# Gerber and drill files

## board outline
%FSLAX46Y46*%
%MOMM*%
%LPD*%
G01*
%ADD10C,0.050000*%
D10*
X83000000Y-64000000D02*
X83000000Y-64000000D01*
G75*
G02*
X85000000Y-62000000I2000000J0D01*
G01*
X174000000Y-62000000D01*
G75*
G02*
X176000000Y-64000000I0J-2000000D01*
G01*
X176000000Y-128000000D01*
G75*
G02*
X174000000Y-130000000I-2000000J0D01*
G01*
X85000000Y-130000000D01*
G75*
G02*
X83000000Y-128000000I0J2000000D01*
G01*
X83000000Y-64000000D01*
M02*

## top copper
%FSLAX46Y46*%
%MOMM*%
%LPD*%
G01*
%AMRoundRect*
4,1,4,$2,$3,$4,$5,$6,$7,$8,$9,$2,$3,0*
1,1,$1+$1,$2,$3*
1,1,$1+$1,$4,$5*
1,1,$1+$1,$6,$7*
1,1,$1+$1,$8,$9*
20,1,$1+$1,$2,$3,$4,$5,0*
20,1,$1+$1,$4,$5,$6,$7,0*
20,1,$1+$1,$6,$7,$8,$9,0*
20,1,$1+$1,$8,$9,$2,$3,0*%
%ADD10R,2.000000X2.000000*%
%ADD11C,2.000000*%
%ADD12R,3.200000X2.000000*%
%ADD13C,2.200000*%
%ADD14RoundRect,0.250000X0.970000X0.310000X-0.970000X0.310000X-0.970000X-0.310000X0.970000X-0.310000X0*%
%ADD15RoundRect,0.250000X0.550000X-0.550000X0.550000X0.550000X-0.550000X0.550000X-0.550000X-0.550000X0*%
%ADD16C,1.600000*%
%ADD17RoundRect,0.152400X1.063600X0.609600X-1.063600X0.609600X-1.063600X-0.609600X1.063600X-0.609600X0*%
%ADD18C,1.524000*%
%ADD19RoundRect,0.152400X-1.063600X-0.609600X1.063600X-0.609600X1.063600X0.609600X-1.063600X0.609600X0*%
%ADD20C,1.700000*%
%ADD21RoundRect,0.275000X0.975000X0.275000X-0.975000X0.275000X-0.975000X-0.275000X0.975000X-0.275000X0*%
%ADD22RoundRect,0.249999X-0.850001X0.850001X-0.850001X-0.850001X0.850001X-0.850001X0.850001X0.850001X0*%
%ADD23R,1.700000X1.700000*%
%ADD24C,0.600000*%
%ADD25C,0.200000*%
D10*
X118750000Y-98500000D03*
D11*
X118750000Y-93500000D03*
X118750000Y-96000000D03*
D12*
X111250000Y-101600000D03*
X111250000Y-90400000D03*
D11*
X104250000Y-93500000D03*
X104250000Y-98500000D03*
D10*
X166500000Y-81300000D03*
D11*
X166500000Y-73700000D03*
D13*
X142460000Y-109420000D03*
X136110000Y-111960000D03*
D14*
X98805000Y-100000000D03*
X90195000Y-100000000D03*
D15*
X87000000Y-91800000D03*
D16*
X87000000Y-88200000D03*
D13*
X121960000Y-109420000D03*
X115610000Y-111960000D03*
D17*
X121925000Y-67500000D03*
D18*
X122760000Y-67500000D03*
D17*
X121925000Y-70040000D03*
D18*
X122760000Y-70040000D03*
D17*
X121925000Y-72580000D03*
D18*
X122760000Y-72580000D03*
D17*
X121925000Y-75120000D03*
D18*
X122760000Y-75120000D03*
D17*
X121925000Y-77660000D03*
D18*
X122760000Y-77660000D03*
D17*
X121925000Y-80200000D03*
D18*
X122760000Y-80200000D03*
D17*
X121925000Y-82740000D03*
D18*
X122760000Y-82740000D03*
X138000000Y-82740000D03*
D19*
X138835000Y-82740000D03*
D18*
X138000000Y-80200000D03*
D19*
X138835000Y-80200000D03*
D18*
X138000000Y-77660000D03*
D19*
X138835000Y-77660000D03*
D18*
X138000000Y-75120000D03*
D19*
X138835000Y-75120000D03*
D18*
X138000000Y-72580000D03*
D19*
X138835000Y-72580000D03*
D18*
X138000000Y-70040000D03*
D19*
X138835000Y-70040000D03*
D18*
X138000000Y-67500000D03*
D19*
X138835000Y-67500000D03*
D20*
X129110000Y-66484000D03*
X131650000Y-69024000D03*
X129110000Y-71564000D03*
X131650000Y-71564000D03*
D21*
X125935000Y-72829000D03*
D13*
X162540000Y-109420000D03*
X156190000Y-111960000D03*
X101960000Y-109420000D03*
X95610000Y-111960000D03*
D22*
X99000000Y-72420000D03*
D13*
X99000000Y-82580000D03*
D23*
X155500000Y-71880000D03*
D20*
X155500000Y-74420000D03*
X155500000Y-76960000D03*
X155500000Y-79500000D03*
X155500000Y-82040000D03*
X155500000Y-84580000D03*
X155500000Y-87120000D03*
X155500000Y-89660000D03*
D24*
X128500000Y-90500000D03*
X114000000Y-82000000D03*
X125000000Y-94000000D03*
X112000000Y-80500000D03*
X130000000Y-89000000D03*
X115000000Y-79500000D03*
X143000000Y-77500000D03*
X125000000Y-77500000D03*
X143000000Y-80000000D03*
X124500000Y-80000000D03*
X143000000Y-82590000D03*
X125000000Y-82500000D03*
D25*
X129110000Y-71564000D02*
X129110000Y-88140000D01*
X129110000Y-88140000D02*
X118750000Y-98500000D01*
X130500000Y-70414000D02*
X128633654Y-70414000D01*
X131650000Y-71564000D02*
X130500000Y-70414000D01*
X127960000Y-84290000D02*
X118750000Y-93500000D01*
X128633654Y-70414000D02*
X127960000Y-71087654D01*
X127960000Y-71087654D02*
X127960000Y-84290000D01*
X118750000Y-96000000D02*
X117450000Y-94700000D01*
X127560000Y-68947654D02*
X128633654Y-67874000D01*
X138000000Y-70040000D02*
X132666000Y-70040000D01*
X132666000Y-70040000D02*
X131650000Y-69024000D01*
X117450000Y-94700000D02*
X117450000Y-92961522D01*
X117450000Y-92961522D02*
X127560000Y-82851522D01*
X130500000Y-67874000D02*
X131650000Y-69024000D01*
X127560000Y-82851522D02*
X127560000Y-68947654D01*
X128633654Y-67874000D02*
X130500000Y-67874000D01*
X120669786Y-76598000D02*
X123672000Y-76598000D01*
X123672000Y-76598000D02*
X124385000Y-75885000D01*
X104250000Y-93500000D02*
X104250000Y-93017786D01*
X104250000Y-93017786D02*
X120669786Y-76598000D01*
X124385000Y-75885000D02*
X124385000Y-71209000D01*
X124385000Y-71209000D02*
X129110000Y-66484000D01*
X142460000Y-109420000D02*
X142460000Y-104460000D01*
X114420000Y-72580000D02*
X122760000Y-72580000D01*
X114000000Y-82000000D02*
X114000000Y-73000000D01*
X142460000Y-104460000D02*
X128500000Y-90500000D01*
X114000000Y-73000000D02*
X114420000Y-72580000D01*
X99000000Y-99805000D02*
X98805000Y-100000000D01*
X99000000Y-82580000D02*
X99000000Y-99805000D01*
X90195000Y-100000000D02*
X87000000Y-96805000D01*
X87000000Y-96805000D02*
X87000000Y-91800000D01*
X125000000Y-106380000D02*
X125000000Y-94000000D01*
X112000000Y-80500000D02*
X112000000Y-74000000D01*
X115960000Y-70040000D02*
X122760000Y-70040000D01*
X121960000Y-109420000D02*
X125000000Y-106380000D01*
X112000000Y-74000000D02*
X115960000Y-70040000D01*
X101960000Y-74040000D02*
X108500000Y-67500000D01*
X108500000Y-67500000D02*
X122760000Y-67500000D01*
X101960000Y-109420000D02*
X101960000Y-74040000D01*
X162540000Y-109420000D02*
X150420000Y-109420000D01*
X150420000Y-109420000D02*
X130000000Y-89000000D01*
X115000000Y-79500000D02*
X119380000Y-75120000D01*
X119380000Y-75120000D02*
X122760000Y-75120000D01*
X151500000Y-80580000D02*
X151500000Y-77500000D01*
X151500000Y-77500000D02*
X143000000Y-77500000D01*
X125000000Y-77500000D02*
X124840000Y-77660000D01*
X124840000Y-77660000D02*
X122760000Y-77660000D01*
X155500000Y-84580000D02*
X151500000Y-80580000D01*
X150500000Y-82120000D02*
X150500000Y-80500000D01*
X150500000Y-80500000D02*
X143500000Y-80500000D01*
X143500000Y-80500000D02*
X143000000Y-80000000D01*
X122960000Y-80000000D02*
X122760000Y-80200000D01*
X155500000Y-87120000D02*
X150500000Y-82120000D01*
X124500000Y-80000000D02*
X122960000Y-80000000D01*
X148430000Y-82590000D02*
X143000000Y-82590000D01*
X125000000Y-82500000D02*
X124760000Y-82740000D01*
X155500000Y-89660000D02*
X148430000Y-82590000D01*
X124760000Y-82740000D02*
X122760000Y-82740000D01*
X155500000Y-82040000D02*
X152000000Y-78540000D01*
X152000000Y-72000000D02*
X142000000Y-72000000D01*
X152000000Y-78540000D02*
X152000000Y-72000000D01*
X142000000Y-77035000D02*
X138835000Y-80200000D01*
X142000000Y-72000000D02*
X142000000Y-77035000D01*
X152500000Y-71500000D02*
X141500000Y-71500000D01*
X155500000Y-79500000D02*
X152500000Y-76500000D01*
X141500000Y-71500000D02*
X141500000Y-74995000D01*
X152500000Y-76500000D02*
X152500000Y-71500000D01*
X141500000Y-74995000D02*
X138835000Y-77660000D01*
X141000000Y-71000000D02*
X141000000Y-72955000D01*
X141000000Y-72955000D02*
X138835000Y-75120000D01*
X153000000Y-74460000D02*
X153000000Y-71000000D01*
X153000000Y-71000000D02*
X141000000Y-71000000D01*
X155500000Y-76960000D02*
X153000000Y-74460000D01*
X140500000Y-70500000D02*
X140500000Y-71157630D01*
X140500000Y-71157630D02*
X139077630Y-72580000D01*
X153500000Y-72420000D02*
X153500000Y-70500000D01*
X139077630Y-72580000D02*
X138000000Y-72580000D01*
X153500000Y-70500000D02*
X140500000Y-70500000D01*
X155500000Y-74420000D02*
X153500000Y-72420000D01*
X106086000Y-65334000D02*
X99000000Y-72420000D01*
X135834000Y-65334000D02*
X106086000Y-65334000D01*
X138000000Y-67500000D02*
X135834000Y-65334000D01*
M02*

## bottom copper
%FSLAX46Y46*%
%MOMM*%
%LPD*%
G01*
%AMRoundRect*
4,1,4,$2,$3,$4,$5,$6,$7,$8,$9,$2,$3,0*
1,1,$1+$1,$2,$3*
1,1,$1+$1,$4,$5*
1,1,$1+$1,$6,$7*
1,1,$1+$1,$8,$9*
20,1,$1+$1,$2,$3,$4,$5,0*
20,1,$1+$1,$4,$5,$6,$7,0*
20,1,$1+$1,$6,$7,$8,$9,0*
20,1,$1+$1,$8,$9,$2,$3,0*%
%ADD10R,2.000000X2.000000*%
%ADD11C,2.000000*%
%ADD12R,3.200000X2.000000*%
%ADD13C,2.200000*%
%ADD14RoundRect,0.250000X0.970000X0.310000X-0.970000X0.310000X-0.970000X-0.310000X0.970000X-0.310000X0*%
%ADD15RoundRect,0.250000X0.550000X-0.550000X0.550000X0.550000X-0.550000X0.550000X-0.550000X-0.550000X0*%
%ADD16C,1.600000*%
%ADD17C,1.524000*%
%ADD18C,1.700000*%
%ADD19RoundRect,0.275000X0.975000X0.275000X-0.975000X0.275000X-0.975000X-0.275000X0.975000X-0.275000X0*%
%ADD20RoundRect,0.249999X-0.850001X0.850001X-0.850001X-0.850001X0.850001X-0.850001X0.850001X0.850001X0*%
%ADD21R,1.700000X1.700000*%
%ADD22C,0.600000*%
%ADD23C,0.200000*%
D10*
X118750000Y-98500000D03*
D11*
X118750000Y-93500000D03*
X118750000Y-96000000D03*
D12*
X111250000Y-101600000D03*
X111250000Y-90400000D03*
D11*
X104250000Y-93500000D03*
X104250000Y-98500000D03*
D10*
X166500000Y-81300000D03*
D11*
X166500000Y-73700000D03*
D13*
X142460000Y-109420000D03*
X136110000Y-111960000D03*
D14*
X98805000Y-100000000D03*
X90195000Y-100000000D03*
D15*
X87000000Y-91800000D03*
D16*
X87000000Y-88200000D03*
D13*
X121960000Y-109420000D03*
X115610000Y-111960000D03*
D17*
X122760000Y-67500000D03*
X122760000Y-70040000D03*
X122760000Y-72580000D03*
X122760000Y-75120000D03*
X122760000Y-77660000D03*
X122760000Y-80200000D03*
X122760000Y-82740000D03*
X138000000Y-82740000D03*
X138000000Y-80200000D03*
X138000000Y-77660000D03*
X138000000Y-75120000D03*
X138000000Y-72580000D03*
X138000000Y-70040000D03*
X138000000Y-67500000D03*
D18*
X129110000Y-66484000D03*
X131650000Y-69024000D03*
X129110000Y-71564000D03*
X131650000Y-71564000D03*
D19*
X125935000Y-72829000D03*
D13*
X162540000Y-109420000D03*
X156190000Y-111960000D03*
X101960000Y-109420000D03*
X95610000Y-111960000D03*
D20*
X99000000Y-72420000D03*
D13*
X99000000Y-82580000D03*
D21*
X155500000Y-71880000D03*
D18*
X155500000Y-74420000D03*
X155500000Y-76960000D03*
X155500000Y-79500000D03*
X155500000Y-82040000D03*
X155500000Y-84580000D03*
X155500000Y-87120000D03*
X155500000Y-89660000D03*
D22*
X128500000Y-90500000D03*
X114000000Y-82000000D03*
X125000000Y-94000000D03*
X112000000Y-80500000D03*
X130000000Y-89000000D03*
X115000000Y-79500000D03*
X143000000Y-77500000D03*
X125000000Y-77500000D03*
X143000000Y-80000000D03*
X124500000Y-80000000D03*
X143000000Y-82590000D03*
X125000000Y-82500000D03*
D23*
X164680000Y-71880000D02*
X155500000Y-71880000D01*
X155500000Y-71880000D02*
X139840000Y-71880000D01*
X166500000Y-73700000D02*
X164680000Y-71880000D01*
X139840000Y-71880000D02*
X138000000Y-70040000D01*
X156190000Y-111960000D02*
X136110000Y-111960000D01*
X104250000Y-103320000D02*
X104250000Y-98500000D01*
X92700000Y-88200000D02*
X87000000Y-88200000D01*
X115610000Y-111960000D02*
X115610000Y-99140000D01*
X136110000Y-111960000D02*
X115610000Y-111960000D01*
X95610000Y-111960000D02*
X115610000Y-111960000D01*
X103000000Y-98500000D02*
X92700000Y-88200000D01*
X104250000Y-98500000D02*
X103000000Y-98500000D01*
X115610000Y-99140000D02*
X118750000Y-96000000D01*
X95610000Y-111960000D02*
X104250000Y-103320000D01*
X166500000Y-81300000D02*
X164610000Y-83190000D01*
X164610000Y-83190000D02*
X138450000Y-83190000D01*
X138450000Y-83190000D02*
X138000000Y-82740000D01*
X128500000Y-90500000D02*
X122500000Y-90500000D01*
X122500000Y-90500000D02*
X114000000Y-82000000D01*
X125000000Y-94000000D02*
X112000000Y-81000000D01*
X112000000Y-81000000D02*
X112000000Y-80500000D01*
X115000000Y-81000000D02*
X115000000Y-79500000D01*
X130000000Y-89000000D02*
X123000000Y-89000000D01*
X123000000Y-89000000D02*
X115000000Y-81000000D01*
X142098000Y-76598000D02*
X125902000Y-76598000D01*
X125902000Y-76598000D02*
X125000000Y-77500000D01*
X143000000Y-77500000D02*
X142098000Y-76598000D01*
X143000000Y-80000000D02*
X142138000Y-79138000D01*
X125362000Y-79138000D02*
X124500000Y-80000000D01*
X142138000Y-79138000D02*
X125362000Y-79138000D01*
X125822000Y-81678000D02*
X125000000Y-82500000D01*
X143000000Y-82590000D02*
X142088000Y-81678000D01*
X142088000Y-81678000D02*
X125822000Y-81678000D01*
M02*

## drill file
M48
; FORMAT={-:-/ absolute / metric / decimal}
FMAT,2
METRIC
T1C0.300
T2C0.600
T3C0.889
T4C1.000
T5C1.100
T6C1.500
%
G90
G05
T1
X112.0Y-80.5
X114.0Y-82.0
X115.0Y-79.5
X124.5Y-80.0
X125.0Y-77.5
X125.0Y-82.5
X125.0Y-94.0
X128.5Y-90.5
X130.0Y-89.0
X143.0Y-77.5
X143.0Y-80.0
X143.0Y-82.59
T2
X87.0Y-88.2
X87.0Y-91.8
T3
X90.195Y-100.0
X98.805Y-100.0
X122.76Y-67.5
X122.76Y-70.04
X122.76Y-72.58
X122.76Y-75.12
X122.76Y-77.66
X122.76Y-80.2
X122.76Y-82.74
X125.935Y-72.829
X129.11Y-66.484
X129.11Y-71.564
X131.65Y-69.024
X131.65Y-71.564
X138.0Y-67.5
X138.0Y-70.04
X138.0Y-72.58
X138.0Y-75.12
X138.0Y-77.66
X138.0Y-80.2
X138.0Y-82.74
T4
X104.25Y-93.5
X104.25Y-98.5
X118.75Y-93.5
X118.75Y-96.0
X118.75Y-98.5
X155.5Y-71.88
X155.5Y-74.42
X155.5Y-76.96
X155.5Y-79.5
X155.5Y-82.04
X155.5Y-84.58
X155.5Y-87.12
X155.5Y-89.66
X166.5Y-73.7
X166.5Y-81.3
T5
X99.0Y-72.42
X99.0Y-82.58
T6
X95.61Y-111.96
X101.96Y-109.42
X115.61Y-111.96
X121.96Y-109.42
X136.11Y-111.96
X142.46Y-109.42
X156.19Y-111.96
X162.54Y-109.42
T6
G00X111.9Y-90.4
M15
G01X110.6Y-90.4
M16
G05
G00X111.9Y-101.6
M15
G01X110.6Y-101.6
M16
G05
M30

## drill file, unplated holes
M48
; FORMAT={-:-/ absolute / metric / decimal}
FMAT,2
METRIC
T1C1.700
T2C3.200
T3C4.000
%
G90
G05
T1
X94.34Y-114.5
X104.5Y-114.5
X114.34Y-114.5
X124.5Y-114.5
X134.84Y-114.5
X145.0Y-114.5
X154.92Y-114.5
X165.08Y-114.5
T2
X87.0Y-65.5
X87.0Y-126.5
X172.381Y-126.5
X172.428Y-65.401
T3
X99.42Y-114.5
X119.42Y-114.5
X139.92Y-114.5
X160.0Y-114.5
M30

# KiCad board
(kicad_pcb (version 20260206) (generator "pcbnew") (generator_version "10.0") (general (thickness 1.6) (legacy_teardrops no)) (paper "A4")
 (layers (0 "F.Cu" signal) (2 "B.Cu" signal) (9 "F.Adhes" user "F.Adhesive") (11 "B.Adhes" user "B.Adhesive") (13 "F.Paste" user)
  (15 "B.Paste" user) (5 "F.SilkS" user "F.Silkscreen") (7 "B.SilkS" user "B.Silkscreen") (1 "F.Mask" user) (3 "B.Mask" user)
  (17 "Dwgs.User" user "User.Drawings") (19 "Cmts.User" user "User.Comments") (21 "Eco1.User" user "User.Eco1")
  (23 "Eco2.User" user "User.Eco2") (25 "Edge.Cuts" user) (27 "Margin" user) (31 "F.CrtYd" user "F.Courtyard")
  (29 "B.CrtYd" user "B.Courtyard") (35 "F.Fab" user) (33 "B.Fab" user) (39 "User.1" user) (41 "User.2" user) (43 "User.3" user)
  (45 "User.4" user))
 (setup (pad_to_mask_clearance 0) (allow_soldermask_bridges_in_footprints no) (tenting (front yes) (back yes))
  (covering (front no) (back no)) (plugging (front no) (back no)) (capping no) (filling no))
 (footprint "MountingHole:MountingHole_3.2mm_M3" (layer "F.Cu") (at 172.380609 126.5)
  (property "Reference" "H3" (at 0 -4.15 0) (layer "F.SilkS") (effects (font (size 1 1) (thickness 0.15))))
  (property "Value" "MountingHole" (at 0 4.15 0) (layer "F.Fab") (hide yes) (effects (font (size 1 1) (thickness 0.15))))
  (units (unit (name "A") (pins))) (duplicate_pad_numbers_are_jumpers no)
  (pad "" np_thru_hole circle (at 0 0) (size 3.2 3.2) (drill 3.2) (layers "*.Cu" "*.Mask")))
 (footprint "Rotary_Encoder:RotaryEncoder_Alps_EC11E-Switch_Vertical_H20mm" (layer "F.Cu") (at 118.75 98.5 180)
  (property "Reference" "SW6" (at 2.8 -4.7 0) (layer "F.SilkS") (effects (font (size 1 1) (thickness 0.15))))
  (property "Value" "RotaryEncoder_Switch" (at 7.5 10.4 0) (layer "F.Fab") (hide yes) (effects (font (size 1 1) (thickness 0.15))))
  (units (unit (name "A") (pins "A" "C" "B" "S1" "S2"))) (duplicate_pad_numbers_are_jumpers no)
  (pad "A" thru_hole rect (at 0 0 180) (size 2 2) (drill 1) (layers "*.Cu" "*.Mask") (remove_unused_layers no)
   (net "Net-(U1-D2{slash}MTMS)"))
  (pad "B" thru_hole circle (at 0 5 180) (size 2 2) (drill 1) (layers "*.Cu" "*.Mask") (remove_unused_layers no)
   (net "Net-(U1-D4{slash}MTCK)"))
  (pad "C" thru_hole circle (at 0 2.5 180) (size 2 2) (drill 1) (layers "*.Cu" "*.Mask") (remove_unused_layers no) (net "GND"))
  (pad "MP" thru_hole rect (at 7.5 -3.1 180) (size 3.2 2) (drill oval 2.8 1.5) (layers "*.Cu" "*.Mask") (remove_unused_layers no))
  (pad "MP" thru_hole rect (at 7.5 8.1 180) (size 3.2 2) (drill oval 2.8 1.5) (layers "*.Cu" "*.Mask") (remove_unused_layers no))
  (pad "S1" thru_hole circle (at 14.5 5 180) (size 2 2) (drill 1) (layers "*.Cu" "*.Mask") (remove_unused_layers no)
   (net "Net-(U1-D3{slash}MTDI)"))
  (pad "S2" thru_hole circle (at 14.5 0 180) (size 2 2) (drill 1) (layers "*.Cu" "*.Mask") (remove_unused_layers no) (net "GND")))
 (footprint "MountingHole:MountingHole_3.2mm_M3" (layer "F.Cu") (at 172.4285 65.401372)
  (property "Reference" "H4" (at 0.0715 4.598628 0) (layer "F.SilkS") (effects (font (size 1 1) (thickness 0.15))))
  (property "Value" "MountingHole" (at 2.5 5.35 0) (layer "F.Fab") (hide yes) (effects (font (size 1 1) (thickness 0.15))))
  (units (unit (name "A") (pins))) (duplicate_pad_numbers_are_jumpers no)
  (pad "" np_thru_hole circle (at 0 0) (size 3.2 3.2) (drill 3.2) (layers "*.Cu" "*.Mask")))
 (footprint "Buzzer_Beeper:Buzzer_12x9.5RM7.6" (layer "F.Cu") (at 166.5 81.3 90)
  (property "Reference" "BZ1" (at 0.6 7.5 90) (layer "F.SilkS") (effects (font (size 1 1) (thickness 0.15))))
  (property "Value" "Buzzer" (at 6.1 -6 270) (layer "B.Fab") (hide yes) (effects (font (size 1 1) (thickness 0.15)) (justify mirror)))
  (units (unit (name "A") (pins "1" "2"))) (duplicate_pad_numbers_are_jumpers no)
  (pad "1" thru_hole rect (at 0 0 90) (size 2 2) (drill 1) (layers "*.Cu" "*.Mask") (remove_unused_layers no) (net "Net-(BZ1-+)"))
  (pad "2" thru_hole circle (at 7.6 0 90) (size 2 2) (drill 1) (layers "*.Cu" "*.Mask") (remove_unused_layers no) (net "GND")))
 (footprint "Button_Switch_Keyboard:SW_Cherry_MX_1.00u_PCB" (layer "F.Cu") (at 142.46 109.42)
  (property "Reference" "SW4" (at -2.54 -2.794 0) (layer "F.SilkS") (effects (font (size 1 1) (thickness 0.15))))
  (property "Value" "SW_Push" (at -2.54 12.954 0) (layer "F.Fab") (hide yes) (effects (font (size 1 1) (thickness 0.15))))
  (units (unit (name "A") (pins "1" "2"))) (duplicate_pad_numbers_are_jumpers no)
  (pad "" np_thru_hole circle (at -7.62 5.08) (size 1.7 1.7) (drill 1.7) (layers "*.Cu" "*.Mask"))
  (pad "" np_thru_hole circle (at -2.54 5.08) (size 4 4) (drill 4) (layers "*.Cu" "*.Mask"))
  (pad "" np_thru_hole circle (at 2.54 5.08) (size 1.7 1.7) (drill 1.7) (layers "*.Cu" "*.Mask"))
  (pad "1" thru_hole circle (at 0 0) (size 2.2 2.2) (drill 1.5) (layers "*.Cu" "*.Mask") (remove_unused_layers no) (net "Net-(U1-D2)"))
  (pad "2" thru_hole circle (at -6.35 2.54) (size 2.2 2.2) (drill 1.5) (layers "*.Cu" "*.Mask") (remove_unused_layers no) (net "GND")))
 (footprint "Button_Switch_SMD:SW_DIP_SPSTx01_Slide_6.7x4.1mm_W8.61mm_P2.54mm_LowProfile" (layer "F.Cu") (at 94.5 100 180)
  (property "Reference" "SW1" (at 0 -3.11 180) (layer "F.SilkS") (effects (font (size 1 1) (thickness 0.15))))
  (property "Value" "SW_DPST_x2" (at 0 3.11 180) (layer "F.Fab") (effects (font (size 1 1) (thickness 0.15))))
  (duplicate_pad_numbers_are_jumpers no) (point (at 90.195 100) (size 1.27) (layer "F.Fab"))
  (pad "1" thru_hole roundrect (at -4.305 0 180) (size 2.44 1.12) (drill 0.889) (layers "*.Cu" "*.Mask" "F.Paste") (remove_unused_layers no)
   (roundrect_rratio 0.223214) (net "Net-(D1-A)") (zone_connect 2))
  (pad "2" thru_hole roundrect (at 4.305 0 180) (size 2.44 1.12) (drill 0.889) (layers "*.Cu" "*.Mask") (remove_unused_layers no)
   (roundrect_rratio 0.223214) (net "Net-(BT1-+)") (zone_connect 2)))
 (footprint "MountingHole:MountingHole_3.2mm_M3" (layer "F.Cu") (at 87 126.5)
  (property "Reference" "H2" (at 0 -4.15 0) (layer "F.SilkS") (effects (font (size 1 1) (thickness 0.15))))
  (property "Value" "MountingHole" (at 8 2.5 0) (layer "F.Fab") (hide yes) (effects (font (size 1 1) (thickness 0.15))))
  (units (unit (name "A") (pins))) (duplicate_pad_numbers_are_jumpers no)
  (pad "" np_thru_hole circle (at 0 0) (size 3.2 3.2) (drill 3.2) (layers "*.Cu" "*.Mask")))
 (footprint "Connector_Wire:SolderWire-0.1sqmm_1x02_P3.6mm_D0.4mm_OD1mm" (layer "F.Cu") (at 87 91.8 90)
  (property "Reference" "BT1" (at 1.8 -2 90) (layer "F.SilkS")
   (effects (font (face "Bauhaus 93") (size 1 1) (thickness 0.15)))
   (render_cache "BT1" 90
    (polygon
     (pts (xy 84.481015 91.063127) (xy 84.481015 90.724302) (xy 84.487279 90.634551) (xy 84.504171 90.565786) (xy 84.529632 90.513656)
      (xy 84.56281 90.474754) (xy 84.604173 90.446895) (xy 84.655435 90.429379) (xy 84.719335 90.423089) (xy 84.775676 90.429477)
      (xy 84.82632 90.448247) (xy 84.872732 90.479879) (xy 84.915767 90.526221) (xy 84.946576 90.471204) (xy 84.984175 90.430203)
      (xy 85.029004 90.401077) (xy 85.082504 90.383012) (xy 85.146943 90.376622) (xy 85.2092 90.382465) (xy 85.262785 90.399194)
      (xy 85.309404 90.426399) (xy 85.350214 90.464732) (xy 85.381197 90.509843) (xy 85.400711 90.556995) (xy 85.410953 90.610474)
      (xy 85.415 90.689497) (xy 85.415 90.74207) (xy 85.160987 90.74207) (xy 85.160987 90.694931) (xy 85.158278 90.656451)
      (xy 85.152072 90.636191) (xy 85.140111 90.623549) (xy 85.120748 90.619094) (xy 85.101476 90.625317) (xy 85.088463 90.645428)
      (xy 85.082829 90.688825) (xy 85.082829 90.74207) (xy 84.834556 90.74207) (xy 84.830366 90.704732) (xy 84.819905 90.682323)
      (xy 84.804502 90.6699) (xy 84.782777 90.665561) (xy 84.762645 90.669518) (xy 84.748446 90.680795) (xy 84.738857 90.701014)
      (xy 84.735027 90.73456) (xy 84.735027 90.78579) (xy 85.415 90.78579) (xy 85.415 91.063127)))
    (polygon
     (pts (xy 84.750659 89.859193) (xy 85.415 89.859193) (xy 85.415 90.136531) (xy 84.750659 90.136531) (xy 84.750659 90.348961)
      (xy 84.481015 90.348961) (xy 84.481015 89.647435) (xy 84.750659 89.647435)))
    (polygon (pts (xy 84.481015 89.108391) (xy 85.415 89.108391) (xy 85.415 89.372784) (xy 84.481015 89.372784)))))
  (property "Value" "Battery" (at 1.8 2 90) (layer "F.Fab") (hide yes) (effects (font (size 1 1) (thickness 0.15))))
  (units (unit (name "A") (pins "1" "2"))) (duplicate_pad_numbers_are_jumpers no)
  (pad "1" thru_hole roundrect (at 0 0 90) (size 1.6 1.6) (drill 0.6) (layers "*.Cu" "*.Mask") (remove_unused_layers no)
   (roundrect_rratio 0.15625) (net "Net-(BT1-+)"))
  (pad "2" thru_hole circle (at 3.6 0 90) (size 1.6 1.6) (drill 0.6) (layers "*.Cu" "*.Mask") (remove_unused_layers no) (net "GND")))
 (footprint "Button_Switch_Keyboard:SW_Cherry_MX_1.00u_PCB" (layer "F.Cu") (at 121.96 109.42)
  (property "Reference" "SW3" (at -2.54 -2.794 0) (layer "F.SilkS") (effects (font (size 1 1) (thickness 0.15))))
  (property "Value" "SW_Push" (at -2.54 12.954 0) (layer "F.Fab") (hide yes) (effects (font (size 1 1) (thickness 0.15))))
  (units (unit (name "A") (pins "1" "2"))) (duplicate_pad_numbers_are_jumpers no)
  (pad "" np_thru_hole circle (at -7.62 5.08) (size 1.7 1.7) (drill 1.7) (layers "*.Cu" "*.Mask"))
  (pad "" np_thru_hole circle (at -2.54 5.08) (size 4 4) (drill 4) (layers "*.Cu" "*.Mask"))
  (pad "" np_thru_hole circle (at 2.54 5.08) (size 1.7 1.7) (drill 1.7) (layers "*.Cu" "*.Mask"))
  (pad "1" thru_hole circle (at 0 0) (size 2.2 2.2) (drill 1.5) (layers "*.Cu" "*.Mask") (remove_unused_layers no) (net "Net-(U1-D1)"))
  (pad "2" thru_hole circle (at -6.35 2.54) (size 2.2 2.2) (drill 1.5) (layers "*.Cu" "*.Mask") (remove_unused_layers no) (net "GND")))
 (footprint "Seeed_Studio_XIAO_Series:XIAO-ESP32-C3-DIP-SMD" (layer "F.Cu") (at 130.38 75.12 90)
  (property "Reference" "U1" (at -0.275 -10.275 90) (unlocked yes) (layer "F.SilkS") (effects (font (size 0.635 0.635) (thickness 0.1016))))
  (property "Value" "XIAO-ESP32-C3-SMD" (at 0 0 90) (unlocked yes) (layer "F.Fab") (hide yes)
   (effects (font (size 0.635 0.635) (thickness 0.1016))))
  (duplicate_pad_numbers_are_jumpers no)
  (pad "1" smd roundrect (at 7.62 -8.455 180) (size 2.432 1.524) (layers "F.Cu" "F.Mask") (roundrect_rratio 0.1) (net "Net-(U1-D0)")
   (thermal_bridge_angle 45))
  (pad "1" thru_hole circle (at 7.62 -7.62 180) (size 1.524 1.524) (drill 0.889) (layers "*.Cu" "*.Mask") (remove_unused_layers no)
   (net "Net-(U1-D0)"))
  (pad "2" smd roundrect (at 5.08 -8.455 180) (size 2.432 1.524) (layers "F.Cu" "F.Mask") (roundrect_rratio 0.1) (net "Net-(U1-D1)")
   (thermal_bridge_angle 45))
  (pad "2" thru_hole circle (at 5.08 -7.62 180) (size 1.524 1.524) (drill 0.889) (layers "*.Cu" "*.Mask") (remove_unused_layers no)
   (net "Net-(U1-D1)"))
  (pad "3" smd roundrect (at 2.54 -8.455 180) (size 2.432 1.524) (layers "F.Cu" "F.Mask") (roundrect_rratio 0.1) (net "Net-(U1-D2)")
   (thermal_bridge_angle 45))
  (pad "3" thru_hole circle (at 2.54 -7.62 180) (size 1.524 1.524) (drill 0.889) (layers "*.Cu" "*.Mask") (remove_unused_layers no)
   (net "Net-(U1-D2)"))
  (pad "4" smd roundrect (at 0 -8.455 180) (size 2.432 1.524) (layers "F.Cu" "F.Mask") (roundrect_rratio 0.1) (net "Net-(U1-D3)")
   (thermal_bridge_angle 45))
  (pad "4" thru_hole circle (at 0 -7.62 180) (size 1.524 1.524) (drill 0.889) (layers "*.Cu" "*.Mask") (remove_unused_layers no)
   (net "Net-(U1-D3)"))
  (pad "5" smd roundrect (at -2.54 -8.455 180) (size 2.432 1.524) (layers "F.Cu" "F.Mask") (roundrect_rratio 0.1) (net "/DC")
   (thermal_bridge_angle 45))
  (pad "5" thru_hole circle (at -2.54 -7.62 180) (size 1.524 1.524) (drill 0.889) (layers "*.Cu" "*.Mask") (remove_unused_layers no)
   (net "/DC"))
  (pad "6" smd roundrect (at -5.08 -8.455 180) (size 2.432 1.524) (layers "F.Cu" "F.Mask") (roundrect_rratio 0.1) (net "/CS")
   (thermal_bridge_angle 45))
  (pad "6" thru_hole circle (at -5.08 -7.62 180) (size 1.524 1.524) (drill 0.889) (layers "*.Cu" "*.Mask") (remove_unused_layers no)
   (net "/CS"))
  (pad "7" smd roundrect (at -7.62 -8.455 180) (size 2.432 1.524) (layers "F.Cu" "F.Mask") (roundrect_rratio 0.1) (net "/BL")
   (thermal_bridge_angle 45))
  (pad "7" thru_hole circle (at -7.62 -7.62 180) (size 1.524 1.524) (drill 0.889) (layers "*.Cu" "*.Mask") (remove_unused_layers no)
   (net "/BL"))
  (pad "8" thru_hole circle (at -7.62 7.62) (size 1.524 1.524) (drill 0.889) (layers "*.Cu" "*.Mask") (remove_unused_layers no)
   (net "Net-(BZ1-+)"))
  (pad "8" smd roundrect (at -7.62 8.455) (size 2.432 1.524) (layers "F.Cu" "F.Mask") (roundrect_rratio 0.1) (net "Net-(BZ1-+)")
   (thermal_bridge_angle 45))
  (pad "9" thru_hole circle (at -5.08 7.62) (size 1.524 1.524) (drill 0.889) (layers "*.Cu" "*.Mask") (remove_unused_layers no) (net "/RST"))
  (pad "9" smd roundrect (at -5.08 8.455) (size 2.432 1.524) (layers "F.Cu" "F.Mask") (roundrect_rratio 0.1) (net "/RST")
   (thermal_bridge_angle 45))
  (pad "10" thru_hole circle (at -2.54 7.62) (size 1.524 1.524) (drill 0.889) (layers "*.Cu" "*.Mask") (remove_unused_layers no)
   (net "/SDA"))
  (pad "10" smd roundrect (at -2.54 8.455) (size 2.432 1.524) (layers "F.Cu" "F.Mask") (roundrect_rratio 0.1) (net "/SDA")
   (thermal_bridge_angle 45))
  (pad "11" thru_hole circle (at 0 7.62) (size 1.524 1.524) (drill 0.889) (layers "*.Cu" "*.Mask") (remove_unused_layers no) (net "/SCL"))
  (pad "11" smd roundrect (at 0 8.455) (size 2.432 1.524) (layers "F.Cu" "F.Mask") (roundrect_rratio 0.1) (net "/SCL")
   (thermal_bridge_angle 45))
  (pad "12" thru_hole circle (at 2.54 7.62) (size 1.524 1.524) (drill 0.889) (layers "*.Cu" "*.Mask") (remove_unused_layers no)
   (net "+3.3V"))
  (pad "12" smd roundrect (at 2.54 8.455) (size 2.432 1.524) (layers "F.Cu" "F.Mask") (roundrect_rratio 0.1) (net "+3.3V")
   (thermal_bridge_angle 45))
  (pad "13" thru_hole circle (at 5.08 7.62) (size 1.524 1.524) (drill 0.889) (layers "*.Cu" "*.Mask") (remove_unused_layers no) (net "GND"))
  (pad "13" smd roundrect (at 5.08 8.455) (size 2.432 1.524) (layers "F.Cu" "F.Mask") (roundrect_rratio 0.1) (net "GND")
   (thermal_bridge_angle 45))
  (pad "14" thru_hole circle (at 7.62 7.62) (size 1.524 1.524) (drill 0.889) (layers "*.Cu" "*.Mask") (remove_unused_layers no)
   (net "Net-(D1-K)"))
  (pad "14" smd roundrect (at 7.62 8.455) (size 2.432 1.524) (layers "F.Cu" "F.Mask") (roundrect_rratio 0.1) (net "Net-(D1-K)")
   (thermal_bridge_angle 45))
  (pad "15" thru_hole circle (at 8.636 -1.27) (size 1.7 1.7) (drill 0.889) (layers "*.Cu" "*.Mask") (remove_unused_layers no)
   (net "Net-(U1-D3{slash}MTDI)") (zone_connect 2))
  (pad "18" thru_hole circle (at 6.096 1.27) (size 1.7 1.7) (drill 0.889) (layers "*.Cu" "*.Mask") (remove_unused_layers no) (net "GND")
   (zone_connect 2))
  (pad "19" thru_hole circle (at 3.556 -1.27) (size 1.7 1.7) (drill 0.889) (layers "*.Cu" "*.Mask") (remove_unused_layers no)
   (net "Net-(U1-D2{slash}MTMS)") (zone_connect 2))
  (pad "20" thru_hole circle (at 3.556 1.27) (size 1.7 1.7) (drill 0.889) (layers "*.Cu" "F.Mask") (remove_unused_layers no)
   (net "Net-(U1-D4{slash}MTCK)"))
  (pad "GND" thru_hole roundrect (at 2.291 -4.445 180) (size 2.5 1.1) (drill 0.889) (layers "*.Cu" "*.Mask") (remove_unused_layers no)
   (roundrect_rratio 0.25) (die_length 2) (thermal_bridge_angle 45)))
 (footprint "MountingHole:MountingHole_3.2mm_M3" (layer "F.Cu") (at 87 65.5)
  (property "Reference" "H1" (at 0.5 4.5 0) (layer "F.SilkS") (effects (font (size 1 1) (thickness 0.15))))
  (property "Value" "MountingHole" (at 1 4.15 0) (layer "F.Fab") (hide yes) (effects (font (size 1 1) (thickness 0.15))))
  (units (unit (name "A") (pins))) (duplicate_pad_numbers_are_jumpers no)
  (pad "" np_thru_hole circle (at 0 0) (size 3.2 3.2) (drill 3.2) (layers "*.Cu" "*.Mask")))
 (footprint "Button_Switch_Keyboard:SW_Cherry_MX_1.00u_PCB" (layer "F.Cu") (at 162.54 109.42)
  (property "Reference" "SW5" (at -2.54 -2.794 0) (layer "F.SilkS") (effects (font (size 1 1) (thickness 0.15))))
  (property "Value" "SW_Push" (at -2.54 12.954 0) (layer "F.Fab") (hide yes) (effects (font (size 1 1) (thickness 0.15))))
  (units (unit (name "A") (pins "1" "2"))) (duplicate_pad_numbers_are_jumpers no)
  (pad "" np_thru_hole circle (at -7.62 5.08) (size 1.7 1.7) (drill 1.7) (layers "*.Cu" "*.Mask"))
  (pad "" np_thru_hole circle (at -2.54 5.08) (size 4 4) (drill 4) (layers "*.Cu" "*.Mask"))
  (pad "" np_thru_hole circle (at 2.54 5.08) (size 1.7 1.7) (drill 1.7) (layers "*.Cu" "*.Mask"))
  (pad "1" thru_hole circle (at 0 0) (size 2.2 2.2) (drill 1.5) (layers "*.Cu" "*.Mask") (remove_unused_layers no) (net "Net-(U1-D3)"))
  (pad "2" thru_hole circle (at -6.35 2.54) (size 2.2 2.2) (drill 1.5) (layers "*.Cu" "*.Mask") (remove_unused_layers no) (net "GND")))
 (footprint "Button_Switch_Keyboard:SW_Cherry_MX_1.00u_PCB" (layer "F.Cu") (at 101.96 109.42)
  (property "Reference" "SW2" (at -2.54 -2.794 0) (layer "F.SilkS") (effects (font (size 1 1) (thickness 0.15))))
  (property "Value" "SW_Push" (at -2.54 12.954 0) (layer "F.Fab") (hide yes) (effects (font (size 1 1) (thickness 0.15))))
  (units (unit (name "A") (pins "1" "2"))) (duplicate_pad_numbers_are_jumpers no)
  (pad "" np_thru_hole circle (at -7.62 5.08) (size 1.7 1.7) (drill 1.7) (layers "*.Cu" "*.Mask"))
  (pad "" np_thru_hole circle (at -2.54 5.08) (size 4 4) (drill 4) (layers "*.Cu" "*.Mask"))
  (pad "" np_thru_hole circle (at 2.54 5.08) (size 1.7 1.7) (drill 1.7) (layers "*.Cu" "*.Mask"))
  (pad "1" thru_hole circle (at 0 0) (size 2.2 2.2) (drill 1.5) (layers "*.Cu" "*.Mask") (remove_unused_layers no) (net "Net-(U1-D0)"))
  (pad "2" thru_hole circle (at -6.35 2.54) (size 2.2 2.2) (drill 1.5) (layers "*.Cu" "*.Mask") (remove_unused_layers no) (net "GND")))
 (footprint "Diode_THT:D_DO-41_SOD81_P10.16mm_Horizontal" (layer "B.Cu") (at 99 72.42 -90)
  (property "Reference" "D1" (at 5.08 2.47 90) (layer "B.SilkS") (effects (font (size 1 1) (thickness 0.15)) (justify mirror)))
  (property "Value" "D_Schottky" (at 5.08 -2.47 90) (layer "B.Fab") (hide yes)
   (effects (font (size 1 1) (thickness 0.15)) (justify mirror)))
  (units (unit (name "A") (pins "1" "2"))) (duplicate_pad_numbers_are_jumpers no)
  (pad "1" thru_hole roundrect (at 0 0 270) (size 2.2 2.2) (drill 1.1) (layers "*.Cu" "*.Mask") (remove_unused_layers no)
   (roundrect_rratio 0.113636) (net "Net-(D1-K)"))
  (pad "2" thru_hole circle (at 10.16 0 270) (size 2.2 2.2) (drill 1.1) (layers "*.Cu" "*.Mask") (remove_unused_layers no)
   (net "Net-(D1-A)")))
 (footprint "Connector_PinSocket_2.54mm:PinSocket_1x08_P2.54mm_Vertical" (layer "B.Cu") (at 155.5 71.88 180)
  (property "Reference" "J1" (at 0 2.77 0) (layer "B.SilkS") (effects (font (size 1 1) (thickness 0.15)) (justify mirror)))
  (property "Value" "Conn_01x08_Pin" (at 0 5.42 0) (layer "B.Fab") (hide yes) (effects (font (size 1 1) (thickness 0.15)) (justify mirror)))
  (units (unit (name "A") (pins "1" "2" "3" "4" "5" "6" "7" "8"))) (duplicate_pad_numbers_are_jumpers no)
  (pad "1" thru_hole rect (at 0 0 180) (size 1.7 1.7) (drill 1) (layers "*.Cu" "*.Mask") (remove_unused_layers no) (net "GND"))
  (pad "2" thru_hole circle (at 0 -2.54 180) (size 1.7 1.7) (drill 1) (layers "*.Cu" "*.Mask") (remove_unused_layers no) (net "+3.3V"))
  (pad "3" thru_hole circle (at 0 -5.08 180) (size 1.7 1.7) (drill 1) (layers "*.Cu" "*.Mask") (remove_unused_layers no) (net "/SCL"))
  (pad "4" thru_hole circle (at 0 -7.62 180) (size 1.7 1.7) (drill 1) (layers "*.Cu" "*.Mask") (remove_unused_layers no) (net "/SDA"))
  (pad "5" thru_hole circle (at 0 -10.16 180) (size 1.7 1.7) (drill 1) (layers "*.Cu" "*.Mask") (remove_unused_layers no) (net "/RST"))
  (pad "6" thru_hole circle (at 0 -12.7 180) (size 1.7 1.7) (drill 1) (layers "*.Cu" "*.Mask") (remove_unused_layers no) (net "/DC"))
  (pad "7" thru_hole circle (at 0 -15.24 180) (size 1.7 1.7) (drill 1) (layers "*.Cu" "*.Mask") (remove_unused_layers no) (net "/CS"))
  (pad "8" thru_hole circle (at 0 -17.78 180) (size 1.7 1.7) (drill 1) (layers "*.Cu" "*.Mask") (remove_unused_layers no) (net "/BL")))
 (gr_rect (start 83 62) (end 176 130) (radius 2) (stroke (width 0.05) (type solid)) (fill no) (layer "Edge.Cuts"))
 (segment (start 129.11 71.564) (end 129.11 88.14) (width 0.2) (layer "F.Cu") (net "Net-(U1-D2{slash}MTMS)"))
 (segment (start 129.11 88.14) (end 118.75 98.5) (width 0.2) (layer "F.Cu") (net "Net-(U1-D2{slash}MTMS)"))
 (segment (start 130.5 70.414) (end 128.633654 70.414) (width 0.2) (layer "F.Cu") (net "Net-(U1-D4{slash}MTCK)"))
 (segment (start 131.65 71.564) (end 130.5 70.414) (width 0.2) (layer "F.Cu") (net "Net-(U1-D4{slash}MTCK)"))
 (segment (start 127.96 84.29) (end 118.75 93.5) (width 0.2) (layer "F.Cu") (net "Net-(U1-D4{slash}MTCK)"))
 (segment (start 128.633654 70.414) (end 127.96 71.087654) (width 0.2) (layer "F.Cu") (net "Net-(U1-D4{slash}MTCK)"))
 (segment (start 127.96 71.087654) (end 127.96 84.29) (width 0.2) (layer "F.Cu") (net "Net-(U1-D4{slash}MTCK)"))
 (segment (start 118.75 96) (end 117.45 94.7) (width 0.2) (layer "F.Cu") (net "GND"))
 (segment (start 127.56 68.947654) (end 128.633654 67.874) (width 0.2) (layer "F.Cu") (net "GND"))
 (segment (start 138 70.04) (end 132.666 70.04) (width 0.2) (layer "F.Cu") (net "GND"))
 (segment (start 132.666 70.04) (end 131.65 69.024) (width 0.2) (layer "F.Cu") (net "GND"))
 (segment (start 117.45 94.7) (end 117.45 92.961522) (width 0.2) (layer "F.Cu") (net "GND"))
 (segment (start 117.45 92.961522) (end 127.56 82.851522) (width 0.2) (layer "F.Cu") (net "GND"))
 (segment (start 130.5 67.874) (end 131.65 69.024) (width 0.2) (layer "F.Cu") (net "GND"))
 (segment (start 127.56 82.851522) (end 127.56 68.947654) (width 0.2) (layer "F.Cu") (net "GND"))
 (segment (start 128.633654 67.874) (end 130.5 67.874) (width 0.2) (layer "F.Cu") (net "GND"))
 (segment (start 164.68 71.88) (end 155.5 71.88) (width 0.2) (layer "B.Cu") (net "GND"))
 (segment (start 155.5 71.88) (end 139.84 71.88) (width 0.2) (layer "B.Cu") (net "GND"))
 (segment (start 166.5 73.7) (end 164.68 71.88) (width 0.2) (layer "B.Cu") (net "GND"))
 (segment (start 139.84 71.88) (end 138 70.04) (width 0.2) (layer "B.Cu") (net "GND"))
 (segment (start 156.19 111.96) (end 136.11 111.96) (width 0.2) (layer "B.Cu") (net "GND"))
 (segment (start 104.25 103.32) (end 104.25 98.5) (width 0.2) (layer "B.Cu") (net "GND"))
 (segment (start 92.7 88.2) (end 87 88.2) (width 0.2) (layer "B.Cu") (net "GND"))
 (segment (start 115.61 111.96) (end 115.61 99.14) (width 0.2) (layer "B.Cu") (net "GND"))
 (segment (start 136.11 111.96) (end 115.61 111.96) (width 0.2) (layer "B.Cu") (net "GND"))
 (segment (start 95.61 111.96) (end 115.61 111.96) (width 0.2) (layer "B.Cu") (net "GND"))
 (segment (start 103 98.5) (end 92.7 88.2) (width 0.2) (layer "B.Cu") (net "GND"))
 (segment (start 104.25 98.5) (end 103 98.5) (width 0.2) (layer "B.Cu") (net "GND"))
 (segment (start 115.61 99.14) (end 118.75 96) (width 0.2) (layer "B.Cu") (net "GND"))
 (segment (start 95.61 111.96) (end 104.25 103.32) (width 0.2) (layer "B.Cu") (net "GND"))
 (segment (start 120.669786 76.598) (end 123.672 76.598) (width 0.2) (layer "F.Cu") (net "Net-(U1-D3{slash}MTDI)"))
 (segment (start 123.672 76.598) (end 124.385 75.885) (width 0.2) (layer "F.Cu") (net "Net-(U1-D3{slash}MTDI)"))
 (segment (start 104.25 93.5) (end 104.25 93.017786) (width 0.2) (layer "F.Cu") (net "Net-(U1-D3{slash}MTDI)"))
 (segment (start 104.25 93.017786) (end 120.669786 76.598) (width 0.2) (layer "F.Cu") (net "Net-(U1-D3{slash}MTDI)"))
 (segment (start 124.385 75.885) (end 124.385 71.209) (width 0.2) (layer "F.Cu") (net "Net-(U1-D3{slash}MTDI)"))
 (segment (start 124.385 71.209) (end 129.11 66.484) (width 0.2) (layer "F.Cu") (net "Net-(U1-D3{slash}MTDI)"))
 (segment (start 166.5 81.3) (end 164.61 83.19) (width 0.2) (layer "B.Cu") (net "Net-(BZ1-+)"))
 (segment (start 164.61 83.19) (end 138.45 83.19) (width 0.2) (layer "B.Cu") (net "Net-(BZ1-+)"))
 (segment (start 138.45 83.19) (end 138 82.74) (width 0.2) (layer "B.Cu") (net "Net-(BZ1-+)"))
 (segment (start 142.46 109.42) (end 142.46 104.46) (width 0.2) (layer "F.Cu") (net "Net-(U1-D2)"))
 (segment (start 114.42 72.58) (end 122.76 72.58) (width 0.2) (layer "F.Cu") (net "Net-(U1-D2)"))
 (segment (start 114 82) (end 114 73) (width 0.2) (layer "F.Cu") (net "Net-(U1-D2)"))
 (segment (start 142.46 104.46) (end 128.5 90.5) (width 0.2) (layer "F.Cu") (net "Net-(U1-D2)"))
 (segment (start 114 73) (end 114.42 72.58) (width 0.2) (layer "F.Cu") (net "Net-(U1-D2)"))
 (via (at 128.5 90.5) (size 0.6) (drill 0.3) (layers "F.Cu" "B.Cu") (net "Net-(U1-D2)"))
 (via (at 114 82) (size 0.6) (drill 0.3) (layers "F.Cu" "B.Cu") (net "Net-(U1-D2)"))
 (segment (start 128.5 90.5) (end 122.5 90.5) (width 0.2) (layer "B.Cu") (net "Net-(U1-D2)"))
 (segment (start 122.5 90.5) (end 114 82) (width 0.2) (layer "B.Cu") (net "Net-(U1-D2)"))
 (segment (start 99 99.805) (end 98.805 100) (width 0.2) (layer "F.Cu") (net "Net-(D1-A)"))
 (segment (start 99 82.58) (end 99 99.805) (width 0.2) (layer "F.Cu") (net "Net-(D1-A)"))
 (segment (start 90.195 100) (end 87 96.805) (width 0.2) (layer "F.Cu") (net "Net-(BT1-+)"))
 (segment (start 87 96.805) (end 87 91.8) (width 0.2) (layer "F.Cu") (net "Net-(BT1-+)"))
 (segment (start 125 106.38) (end 125 94) (width 0.2) (layer "F.Cu") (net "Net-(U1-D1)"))
 (segment (start 112 80.5) (end 112 74) (width 0.2) (layer "F.Cu") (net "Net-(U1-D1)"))
 (segment (start 115.96 70.04) (end 122.76 70.04) (width 0.2) (layer "F.Cu") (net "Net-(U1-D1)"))
 (segment (start 121.96 109.42) (end 125 106.38) (width 0.2) (layer "F.Cu") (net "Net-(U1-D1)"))
 (segment (start 112 74) (end 115.96 70.04) (width 0.2) (layer "F.Cu") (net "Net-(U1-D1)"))
 (via (at 125 94) (size 0.6) (drill 0.3) (layers "F.Cu" "B.Cu") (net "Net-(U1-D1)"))
 (via (at 112 80.5) (size 0.6) (drill 0.3) (layers "F.Cu" "B.Cu") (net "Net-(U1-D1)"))
 (segment (start 125 94) (end 112 81) (width 0.2) (layer "B.Cu") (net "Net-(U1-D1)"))
 (segment (start 112 81) (end 112 80.5) (width 0.2) (layer "B.Cu") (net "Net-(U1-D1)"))
 (segment (start 101.96 74.04) (end 108.5 67.5) (width 0.2) (layer "F.Cu") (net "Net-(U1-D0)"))
 (segment (start 108.5 67.5) (end 122.76 67.5) (width 0.2) (layer "F.Cu") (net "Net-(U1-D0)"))
 (segment (start 101.96 109.42) (end 101.96 74.04) (width 0.2) (layer "F.Cu") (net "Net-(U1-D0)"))
 (segment (start 162.54 109.42) (end 150.42 109.42) (width 0.2) (layer "F.Cu") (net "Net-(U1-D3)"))
 (segment (start 150.42 109.42) (end 130 89) (width 0.2) (layer "F.Cu") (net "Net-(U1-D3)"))
 (segment (start 115 79.5) (end 119.38 75.12) (width 0.2) (layer "F.Cu") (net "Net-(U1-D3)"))
 (segment (start 119.38 75.12) (end 122.76 75.12) (width 0.2) (layer "F.Cu") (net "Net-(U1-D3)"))
 (via (at 130 89) (size 0.6) (drill 0.3) (layers "F.Cu" "B.Cu") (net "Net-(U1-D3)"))
 (via (at 115 79.5) (size 0.6) (drill 0.3) (layers "F.Cu" "B.Cu") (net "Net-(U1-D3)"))
 (segment (start 115 81) (end 115 79.5) (width 0.2) (layer "B.Cu") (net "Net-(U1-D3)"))
 (segment (start 130 89) (end 123 89) (width 0.2) (layer "B.Cu") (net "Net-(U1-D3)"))
 (segment (start 123 89) (end 115 81) (width 0.2) (layer "B.Cu") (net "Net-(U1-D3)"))
 (segment (start 151.5 80.58) (end 151.5 77.5) (width 0.2) (layer "F.Cu") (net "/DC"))
 (segment (start 151.5 77.5) (end 143 77.5) (width 0.2) (layer "F.Cu") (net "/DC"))
 (segment (start 125 77.5) (end 124.84 77.66) (width 0.2) (layer "F.Cu") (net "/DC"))
 (segment (start 124.84 77.66) (end 122.76 77.66) (width 0.2) (layer "F.Cu") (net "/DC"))
 (segment (start 155.5 84.58) (end 151.5 80.58) (width 0.2) (layer "F.Cu") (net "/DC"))
 (via (at 143 77.5) (size 0.6) (drill 0.3) (layers "F.Cu" "B.Cu") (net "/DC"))
 (via (at 125 77.5) (size 0.6) (drill 0.3) (layers "F.Cu" "B.Cu") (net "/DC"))
 (segment (start 142.098 76.598) (end 125.902 76.598) (width 0.2) (layer "B.Cu") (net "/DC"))
 (segment (start 125.902 76.598) (end 125 77.5) (width 0.2) (layer "B.Cu") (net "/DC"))
 (segment (start 143 77.5) (end 142.098 76.598) (width 0.2) (layer "B.Cu") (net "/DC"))
 (segment (start 150.5 82.12) (end 150.5 80.5) (width 0.2) (layer "F.Cu") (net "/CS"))
 (segment (start 150.5 80.5) (end 143.5 80.5) (width 0.2) (layer "F.Cu") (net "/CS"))
 (segment (start 143.5 80.5) (end 143 80) (width 0.2) (layer "F.Cu") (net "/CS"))
 (segment (start 122.96 80) (end 122.76 80.2) (width 0.2) (layer "F.Cu") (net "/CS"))
 (segment (start 155.5 87.12) (end 150.5 82.12) (width 0.2) (layer "F.Cu") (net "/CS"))
 (segment (start 124.5 80) (end 122.96 80) (width 0.2) (layer "F.Cu") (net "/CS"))
 (via (at 143 80) (size 0.6) (drill 0.3) (layers "F.Cu" "B.Cu") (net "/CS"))
 (via (at 124.5 80) (size 0.6) (drill 0.3) (layers "F.Cu" "B.Cu") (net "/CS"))
 (segment (start 143 80) (end 142.138 79.138) (width 0.2) (layer "B.Cu") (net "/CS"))
 (segment (start 125.362 79.138) (end 124.5 80) (width 0.2) (layer "B.Cu") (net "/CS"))
 (segment (start 142.138 79.138) (end 125.362 79.138) (width 0.2) (layer "B.Cu") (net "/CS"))
 (segment (start 148.43 82.59) (end 143 82.59) (width 0.2) (layer "F.Cu") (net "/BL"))
 (segment (start 125 82.5) (end 124.76 82.74) (width 0.2) (layer "F.Cu") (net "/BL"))
 (segment (start 155.5 89.66) (end 148.43 82.59) (width 0.2) (layer "F.Cu") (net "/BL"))
 (segment (start 124.76 82.74) (end 122.76 82.74) (width 0.2) (layer "F.Cu") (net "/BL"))
 (via (at 143 82.59) (size 0.6) (drill 0.3) (layers "F.Cu" "B.Cu") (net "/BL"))
 (via (at 125 82.5) (size 0.6) (drill 0.3) (layers "F.Cu" "B.Cu") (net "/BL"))
 (segment (start 125.822 81.678) (end 125 82.5) (width 0.2) (layer "B.Cu") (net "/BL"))
 (segment (start 143 82.59) (end 142.088 81.678) (width 0.2) (layer "B.Cu") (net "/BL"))
 (segment (start 142.088 81.678) (end 125.822 81.678) (width 0.2) (layer "B.Cu") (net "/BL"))
 (segment (start 155.5 82.04) (end 152 78.54) (width 0.2) (layer "F.Cu") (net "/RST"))
 (segment (start 152 72) (end 142 72) (width 0.2) (layer "F.Cu") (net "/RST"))
 (segment (start 152 78.54) (end 152 72) (width 0.2) (layer "F.Cu") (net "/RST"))
 (segment (start 142 77.035) (end 138.835 80.2) (width 0.2) (layer "F.Cu") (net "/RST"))
 (segment (start 142 72) (end 142 77.035) (width 0.2) (layer "F.Cu") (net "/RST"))
 (segment (start 152.5 71.5) (end 141.5 71.5) (width 0.2) (layer "F.Cu") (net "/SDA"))
 (segment (start 155.5 79.5) (end 152.5 76.5) (width 0.2) (layer "F.Cu") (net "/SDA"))
 (segment (start 141.5 71.5) (end 141.5 74.995) (width 0.2) (layer "F.Cu") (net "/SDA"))
 (segment (start 152.5 76.5) (end 152.5 71.5) (width 0.2) (layer "F.Cu") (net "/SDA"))
 (segment (start 141.5 74.995) (end 138.835 77.66) (width 0.2) (layer "F.Cu") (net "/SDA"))
 (segment (start 141 71) (end 141 72.955) (width 0.2) (layer "F.Cu") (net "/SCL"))
 (segment (start 141 72.955) (end 138.835 75.12) (width 0.2) (layer "F.Cu") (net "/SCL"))
 (segment (start 153 74.46) (end 153 71) (width 0.2) (layer "F.Cu") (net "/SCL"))
 (segment (start 153 71) (end 141 71) (width 0.2) (layer "F.Cu") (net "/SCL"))
 (segment (start 155.5 76.96) (end 153 74.46) (width 0.2) (layer "F.Cu") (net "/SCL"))
 (segment (start 140.5 70.5) (end 140.5 71.15763) (width 0.2) (layer "F.Cu") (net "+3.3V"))
 (segment (start 140.5 71.15763) (end 139.07763 72.58) (width 0.2) (layer "F.Cu") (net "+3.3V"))
 (segment (start 153.5 72.42) (end 153.5 70.5) (width 0.2) (layer "F.Cu") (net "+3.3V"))
 (segment (start 139.07763 72.58) (end 138 72.58) (width 0.2) (layer "F.Cu") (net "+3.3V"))
 (segment (start 153.5 70.5) (end 140.5 70.5) (width 0.2) (layer "F.Cu") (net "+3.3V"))
 (segment (start 155.5 74.42) (end 153.5 72.42) (width 0.2) (layer "F.Cu") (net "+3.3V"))
 (segment (start 106.086 65.334) (end 99 72.42) (width 0.2) (layer "F.Cu") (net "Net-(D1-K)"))
 (segment (start 135.834 65.334) (end 106.086 65.334) (width 0.2) (layer "F.Cu") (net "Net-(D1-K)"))
 (segment (start 138 67.5) (end 135.834 65.334) (width 0.2) (layer "F.Cu") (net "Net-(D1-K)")))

